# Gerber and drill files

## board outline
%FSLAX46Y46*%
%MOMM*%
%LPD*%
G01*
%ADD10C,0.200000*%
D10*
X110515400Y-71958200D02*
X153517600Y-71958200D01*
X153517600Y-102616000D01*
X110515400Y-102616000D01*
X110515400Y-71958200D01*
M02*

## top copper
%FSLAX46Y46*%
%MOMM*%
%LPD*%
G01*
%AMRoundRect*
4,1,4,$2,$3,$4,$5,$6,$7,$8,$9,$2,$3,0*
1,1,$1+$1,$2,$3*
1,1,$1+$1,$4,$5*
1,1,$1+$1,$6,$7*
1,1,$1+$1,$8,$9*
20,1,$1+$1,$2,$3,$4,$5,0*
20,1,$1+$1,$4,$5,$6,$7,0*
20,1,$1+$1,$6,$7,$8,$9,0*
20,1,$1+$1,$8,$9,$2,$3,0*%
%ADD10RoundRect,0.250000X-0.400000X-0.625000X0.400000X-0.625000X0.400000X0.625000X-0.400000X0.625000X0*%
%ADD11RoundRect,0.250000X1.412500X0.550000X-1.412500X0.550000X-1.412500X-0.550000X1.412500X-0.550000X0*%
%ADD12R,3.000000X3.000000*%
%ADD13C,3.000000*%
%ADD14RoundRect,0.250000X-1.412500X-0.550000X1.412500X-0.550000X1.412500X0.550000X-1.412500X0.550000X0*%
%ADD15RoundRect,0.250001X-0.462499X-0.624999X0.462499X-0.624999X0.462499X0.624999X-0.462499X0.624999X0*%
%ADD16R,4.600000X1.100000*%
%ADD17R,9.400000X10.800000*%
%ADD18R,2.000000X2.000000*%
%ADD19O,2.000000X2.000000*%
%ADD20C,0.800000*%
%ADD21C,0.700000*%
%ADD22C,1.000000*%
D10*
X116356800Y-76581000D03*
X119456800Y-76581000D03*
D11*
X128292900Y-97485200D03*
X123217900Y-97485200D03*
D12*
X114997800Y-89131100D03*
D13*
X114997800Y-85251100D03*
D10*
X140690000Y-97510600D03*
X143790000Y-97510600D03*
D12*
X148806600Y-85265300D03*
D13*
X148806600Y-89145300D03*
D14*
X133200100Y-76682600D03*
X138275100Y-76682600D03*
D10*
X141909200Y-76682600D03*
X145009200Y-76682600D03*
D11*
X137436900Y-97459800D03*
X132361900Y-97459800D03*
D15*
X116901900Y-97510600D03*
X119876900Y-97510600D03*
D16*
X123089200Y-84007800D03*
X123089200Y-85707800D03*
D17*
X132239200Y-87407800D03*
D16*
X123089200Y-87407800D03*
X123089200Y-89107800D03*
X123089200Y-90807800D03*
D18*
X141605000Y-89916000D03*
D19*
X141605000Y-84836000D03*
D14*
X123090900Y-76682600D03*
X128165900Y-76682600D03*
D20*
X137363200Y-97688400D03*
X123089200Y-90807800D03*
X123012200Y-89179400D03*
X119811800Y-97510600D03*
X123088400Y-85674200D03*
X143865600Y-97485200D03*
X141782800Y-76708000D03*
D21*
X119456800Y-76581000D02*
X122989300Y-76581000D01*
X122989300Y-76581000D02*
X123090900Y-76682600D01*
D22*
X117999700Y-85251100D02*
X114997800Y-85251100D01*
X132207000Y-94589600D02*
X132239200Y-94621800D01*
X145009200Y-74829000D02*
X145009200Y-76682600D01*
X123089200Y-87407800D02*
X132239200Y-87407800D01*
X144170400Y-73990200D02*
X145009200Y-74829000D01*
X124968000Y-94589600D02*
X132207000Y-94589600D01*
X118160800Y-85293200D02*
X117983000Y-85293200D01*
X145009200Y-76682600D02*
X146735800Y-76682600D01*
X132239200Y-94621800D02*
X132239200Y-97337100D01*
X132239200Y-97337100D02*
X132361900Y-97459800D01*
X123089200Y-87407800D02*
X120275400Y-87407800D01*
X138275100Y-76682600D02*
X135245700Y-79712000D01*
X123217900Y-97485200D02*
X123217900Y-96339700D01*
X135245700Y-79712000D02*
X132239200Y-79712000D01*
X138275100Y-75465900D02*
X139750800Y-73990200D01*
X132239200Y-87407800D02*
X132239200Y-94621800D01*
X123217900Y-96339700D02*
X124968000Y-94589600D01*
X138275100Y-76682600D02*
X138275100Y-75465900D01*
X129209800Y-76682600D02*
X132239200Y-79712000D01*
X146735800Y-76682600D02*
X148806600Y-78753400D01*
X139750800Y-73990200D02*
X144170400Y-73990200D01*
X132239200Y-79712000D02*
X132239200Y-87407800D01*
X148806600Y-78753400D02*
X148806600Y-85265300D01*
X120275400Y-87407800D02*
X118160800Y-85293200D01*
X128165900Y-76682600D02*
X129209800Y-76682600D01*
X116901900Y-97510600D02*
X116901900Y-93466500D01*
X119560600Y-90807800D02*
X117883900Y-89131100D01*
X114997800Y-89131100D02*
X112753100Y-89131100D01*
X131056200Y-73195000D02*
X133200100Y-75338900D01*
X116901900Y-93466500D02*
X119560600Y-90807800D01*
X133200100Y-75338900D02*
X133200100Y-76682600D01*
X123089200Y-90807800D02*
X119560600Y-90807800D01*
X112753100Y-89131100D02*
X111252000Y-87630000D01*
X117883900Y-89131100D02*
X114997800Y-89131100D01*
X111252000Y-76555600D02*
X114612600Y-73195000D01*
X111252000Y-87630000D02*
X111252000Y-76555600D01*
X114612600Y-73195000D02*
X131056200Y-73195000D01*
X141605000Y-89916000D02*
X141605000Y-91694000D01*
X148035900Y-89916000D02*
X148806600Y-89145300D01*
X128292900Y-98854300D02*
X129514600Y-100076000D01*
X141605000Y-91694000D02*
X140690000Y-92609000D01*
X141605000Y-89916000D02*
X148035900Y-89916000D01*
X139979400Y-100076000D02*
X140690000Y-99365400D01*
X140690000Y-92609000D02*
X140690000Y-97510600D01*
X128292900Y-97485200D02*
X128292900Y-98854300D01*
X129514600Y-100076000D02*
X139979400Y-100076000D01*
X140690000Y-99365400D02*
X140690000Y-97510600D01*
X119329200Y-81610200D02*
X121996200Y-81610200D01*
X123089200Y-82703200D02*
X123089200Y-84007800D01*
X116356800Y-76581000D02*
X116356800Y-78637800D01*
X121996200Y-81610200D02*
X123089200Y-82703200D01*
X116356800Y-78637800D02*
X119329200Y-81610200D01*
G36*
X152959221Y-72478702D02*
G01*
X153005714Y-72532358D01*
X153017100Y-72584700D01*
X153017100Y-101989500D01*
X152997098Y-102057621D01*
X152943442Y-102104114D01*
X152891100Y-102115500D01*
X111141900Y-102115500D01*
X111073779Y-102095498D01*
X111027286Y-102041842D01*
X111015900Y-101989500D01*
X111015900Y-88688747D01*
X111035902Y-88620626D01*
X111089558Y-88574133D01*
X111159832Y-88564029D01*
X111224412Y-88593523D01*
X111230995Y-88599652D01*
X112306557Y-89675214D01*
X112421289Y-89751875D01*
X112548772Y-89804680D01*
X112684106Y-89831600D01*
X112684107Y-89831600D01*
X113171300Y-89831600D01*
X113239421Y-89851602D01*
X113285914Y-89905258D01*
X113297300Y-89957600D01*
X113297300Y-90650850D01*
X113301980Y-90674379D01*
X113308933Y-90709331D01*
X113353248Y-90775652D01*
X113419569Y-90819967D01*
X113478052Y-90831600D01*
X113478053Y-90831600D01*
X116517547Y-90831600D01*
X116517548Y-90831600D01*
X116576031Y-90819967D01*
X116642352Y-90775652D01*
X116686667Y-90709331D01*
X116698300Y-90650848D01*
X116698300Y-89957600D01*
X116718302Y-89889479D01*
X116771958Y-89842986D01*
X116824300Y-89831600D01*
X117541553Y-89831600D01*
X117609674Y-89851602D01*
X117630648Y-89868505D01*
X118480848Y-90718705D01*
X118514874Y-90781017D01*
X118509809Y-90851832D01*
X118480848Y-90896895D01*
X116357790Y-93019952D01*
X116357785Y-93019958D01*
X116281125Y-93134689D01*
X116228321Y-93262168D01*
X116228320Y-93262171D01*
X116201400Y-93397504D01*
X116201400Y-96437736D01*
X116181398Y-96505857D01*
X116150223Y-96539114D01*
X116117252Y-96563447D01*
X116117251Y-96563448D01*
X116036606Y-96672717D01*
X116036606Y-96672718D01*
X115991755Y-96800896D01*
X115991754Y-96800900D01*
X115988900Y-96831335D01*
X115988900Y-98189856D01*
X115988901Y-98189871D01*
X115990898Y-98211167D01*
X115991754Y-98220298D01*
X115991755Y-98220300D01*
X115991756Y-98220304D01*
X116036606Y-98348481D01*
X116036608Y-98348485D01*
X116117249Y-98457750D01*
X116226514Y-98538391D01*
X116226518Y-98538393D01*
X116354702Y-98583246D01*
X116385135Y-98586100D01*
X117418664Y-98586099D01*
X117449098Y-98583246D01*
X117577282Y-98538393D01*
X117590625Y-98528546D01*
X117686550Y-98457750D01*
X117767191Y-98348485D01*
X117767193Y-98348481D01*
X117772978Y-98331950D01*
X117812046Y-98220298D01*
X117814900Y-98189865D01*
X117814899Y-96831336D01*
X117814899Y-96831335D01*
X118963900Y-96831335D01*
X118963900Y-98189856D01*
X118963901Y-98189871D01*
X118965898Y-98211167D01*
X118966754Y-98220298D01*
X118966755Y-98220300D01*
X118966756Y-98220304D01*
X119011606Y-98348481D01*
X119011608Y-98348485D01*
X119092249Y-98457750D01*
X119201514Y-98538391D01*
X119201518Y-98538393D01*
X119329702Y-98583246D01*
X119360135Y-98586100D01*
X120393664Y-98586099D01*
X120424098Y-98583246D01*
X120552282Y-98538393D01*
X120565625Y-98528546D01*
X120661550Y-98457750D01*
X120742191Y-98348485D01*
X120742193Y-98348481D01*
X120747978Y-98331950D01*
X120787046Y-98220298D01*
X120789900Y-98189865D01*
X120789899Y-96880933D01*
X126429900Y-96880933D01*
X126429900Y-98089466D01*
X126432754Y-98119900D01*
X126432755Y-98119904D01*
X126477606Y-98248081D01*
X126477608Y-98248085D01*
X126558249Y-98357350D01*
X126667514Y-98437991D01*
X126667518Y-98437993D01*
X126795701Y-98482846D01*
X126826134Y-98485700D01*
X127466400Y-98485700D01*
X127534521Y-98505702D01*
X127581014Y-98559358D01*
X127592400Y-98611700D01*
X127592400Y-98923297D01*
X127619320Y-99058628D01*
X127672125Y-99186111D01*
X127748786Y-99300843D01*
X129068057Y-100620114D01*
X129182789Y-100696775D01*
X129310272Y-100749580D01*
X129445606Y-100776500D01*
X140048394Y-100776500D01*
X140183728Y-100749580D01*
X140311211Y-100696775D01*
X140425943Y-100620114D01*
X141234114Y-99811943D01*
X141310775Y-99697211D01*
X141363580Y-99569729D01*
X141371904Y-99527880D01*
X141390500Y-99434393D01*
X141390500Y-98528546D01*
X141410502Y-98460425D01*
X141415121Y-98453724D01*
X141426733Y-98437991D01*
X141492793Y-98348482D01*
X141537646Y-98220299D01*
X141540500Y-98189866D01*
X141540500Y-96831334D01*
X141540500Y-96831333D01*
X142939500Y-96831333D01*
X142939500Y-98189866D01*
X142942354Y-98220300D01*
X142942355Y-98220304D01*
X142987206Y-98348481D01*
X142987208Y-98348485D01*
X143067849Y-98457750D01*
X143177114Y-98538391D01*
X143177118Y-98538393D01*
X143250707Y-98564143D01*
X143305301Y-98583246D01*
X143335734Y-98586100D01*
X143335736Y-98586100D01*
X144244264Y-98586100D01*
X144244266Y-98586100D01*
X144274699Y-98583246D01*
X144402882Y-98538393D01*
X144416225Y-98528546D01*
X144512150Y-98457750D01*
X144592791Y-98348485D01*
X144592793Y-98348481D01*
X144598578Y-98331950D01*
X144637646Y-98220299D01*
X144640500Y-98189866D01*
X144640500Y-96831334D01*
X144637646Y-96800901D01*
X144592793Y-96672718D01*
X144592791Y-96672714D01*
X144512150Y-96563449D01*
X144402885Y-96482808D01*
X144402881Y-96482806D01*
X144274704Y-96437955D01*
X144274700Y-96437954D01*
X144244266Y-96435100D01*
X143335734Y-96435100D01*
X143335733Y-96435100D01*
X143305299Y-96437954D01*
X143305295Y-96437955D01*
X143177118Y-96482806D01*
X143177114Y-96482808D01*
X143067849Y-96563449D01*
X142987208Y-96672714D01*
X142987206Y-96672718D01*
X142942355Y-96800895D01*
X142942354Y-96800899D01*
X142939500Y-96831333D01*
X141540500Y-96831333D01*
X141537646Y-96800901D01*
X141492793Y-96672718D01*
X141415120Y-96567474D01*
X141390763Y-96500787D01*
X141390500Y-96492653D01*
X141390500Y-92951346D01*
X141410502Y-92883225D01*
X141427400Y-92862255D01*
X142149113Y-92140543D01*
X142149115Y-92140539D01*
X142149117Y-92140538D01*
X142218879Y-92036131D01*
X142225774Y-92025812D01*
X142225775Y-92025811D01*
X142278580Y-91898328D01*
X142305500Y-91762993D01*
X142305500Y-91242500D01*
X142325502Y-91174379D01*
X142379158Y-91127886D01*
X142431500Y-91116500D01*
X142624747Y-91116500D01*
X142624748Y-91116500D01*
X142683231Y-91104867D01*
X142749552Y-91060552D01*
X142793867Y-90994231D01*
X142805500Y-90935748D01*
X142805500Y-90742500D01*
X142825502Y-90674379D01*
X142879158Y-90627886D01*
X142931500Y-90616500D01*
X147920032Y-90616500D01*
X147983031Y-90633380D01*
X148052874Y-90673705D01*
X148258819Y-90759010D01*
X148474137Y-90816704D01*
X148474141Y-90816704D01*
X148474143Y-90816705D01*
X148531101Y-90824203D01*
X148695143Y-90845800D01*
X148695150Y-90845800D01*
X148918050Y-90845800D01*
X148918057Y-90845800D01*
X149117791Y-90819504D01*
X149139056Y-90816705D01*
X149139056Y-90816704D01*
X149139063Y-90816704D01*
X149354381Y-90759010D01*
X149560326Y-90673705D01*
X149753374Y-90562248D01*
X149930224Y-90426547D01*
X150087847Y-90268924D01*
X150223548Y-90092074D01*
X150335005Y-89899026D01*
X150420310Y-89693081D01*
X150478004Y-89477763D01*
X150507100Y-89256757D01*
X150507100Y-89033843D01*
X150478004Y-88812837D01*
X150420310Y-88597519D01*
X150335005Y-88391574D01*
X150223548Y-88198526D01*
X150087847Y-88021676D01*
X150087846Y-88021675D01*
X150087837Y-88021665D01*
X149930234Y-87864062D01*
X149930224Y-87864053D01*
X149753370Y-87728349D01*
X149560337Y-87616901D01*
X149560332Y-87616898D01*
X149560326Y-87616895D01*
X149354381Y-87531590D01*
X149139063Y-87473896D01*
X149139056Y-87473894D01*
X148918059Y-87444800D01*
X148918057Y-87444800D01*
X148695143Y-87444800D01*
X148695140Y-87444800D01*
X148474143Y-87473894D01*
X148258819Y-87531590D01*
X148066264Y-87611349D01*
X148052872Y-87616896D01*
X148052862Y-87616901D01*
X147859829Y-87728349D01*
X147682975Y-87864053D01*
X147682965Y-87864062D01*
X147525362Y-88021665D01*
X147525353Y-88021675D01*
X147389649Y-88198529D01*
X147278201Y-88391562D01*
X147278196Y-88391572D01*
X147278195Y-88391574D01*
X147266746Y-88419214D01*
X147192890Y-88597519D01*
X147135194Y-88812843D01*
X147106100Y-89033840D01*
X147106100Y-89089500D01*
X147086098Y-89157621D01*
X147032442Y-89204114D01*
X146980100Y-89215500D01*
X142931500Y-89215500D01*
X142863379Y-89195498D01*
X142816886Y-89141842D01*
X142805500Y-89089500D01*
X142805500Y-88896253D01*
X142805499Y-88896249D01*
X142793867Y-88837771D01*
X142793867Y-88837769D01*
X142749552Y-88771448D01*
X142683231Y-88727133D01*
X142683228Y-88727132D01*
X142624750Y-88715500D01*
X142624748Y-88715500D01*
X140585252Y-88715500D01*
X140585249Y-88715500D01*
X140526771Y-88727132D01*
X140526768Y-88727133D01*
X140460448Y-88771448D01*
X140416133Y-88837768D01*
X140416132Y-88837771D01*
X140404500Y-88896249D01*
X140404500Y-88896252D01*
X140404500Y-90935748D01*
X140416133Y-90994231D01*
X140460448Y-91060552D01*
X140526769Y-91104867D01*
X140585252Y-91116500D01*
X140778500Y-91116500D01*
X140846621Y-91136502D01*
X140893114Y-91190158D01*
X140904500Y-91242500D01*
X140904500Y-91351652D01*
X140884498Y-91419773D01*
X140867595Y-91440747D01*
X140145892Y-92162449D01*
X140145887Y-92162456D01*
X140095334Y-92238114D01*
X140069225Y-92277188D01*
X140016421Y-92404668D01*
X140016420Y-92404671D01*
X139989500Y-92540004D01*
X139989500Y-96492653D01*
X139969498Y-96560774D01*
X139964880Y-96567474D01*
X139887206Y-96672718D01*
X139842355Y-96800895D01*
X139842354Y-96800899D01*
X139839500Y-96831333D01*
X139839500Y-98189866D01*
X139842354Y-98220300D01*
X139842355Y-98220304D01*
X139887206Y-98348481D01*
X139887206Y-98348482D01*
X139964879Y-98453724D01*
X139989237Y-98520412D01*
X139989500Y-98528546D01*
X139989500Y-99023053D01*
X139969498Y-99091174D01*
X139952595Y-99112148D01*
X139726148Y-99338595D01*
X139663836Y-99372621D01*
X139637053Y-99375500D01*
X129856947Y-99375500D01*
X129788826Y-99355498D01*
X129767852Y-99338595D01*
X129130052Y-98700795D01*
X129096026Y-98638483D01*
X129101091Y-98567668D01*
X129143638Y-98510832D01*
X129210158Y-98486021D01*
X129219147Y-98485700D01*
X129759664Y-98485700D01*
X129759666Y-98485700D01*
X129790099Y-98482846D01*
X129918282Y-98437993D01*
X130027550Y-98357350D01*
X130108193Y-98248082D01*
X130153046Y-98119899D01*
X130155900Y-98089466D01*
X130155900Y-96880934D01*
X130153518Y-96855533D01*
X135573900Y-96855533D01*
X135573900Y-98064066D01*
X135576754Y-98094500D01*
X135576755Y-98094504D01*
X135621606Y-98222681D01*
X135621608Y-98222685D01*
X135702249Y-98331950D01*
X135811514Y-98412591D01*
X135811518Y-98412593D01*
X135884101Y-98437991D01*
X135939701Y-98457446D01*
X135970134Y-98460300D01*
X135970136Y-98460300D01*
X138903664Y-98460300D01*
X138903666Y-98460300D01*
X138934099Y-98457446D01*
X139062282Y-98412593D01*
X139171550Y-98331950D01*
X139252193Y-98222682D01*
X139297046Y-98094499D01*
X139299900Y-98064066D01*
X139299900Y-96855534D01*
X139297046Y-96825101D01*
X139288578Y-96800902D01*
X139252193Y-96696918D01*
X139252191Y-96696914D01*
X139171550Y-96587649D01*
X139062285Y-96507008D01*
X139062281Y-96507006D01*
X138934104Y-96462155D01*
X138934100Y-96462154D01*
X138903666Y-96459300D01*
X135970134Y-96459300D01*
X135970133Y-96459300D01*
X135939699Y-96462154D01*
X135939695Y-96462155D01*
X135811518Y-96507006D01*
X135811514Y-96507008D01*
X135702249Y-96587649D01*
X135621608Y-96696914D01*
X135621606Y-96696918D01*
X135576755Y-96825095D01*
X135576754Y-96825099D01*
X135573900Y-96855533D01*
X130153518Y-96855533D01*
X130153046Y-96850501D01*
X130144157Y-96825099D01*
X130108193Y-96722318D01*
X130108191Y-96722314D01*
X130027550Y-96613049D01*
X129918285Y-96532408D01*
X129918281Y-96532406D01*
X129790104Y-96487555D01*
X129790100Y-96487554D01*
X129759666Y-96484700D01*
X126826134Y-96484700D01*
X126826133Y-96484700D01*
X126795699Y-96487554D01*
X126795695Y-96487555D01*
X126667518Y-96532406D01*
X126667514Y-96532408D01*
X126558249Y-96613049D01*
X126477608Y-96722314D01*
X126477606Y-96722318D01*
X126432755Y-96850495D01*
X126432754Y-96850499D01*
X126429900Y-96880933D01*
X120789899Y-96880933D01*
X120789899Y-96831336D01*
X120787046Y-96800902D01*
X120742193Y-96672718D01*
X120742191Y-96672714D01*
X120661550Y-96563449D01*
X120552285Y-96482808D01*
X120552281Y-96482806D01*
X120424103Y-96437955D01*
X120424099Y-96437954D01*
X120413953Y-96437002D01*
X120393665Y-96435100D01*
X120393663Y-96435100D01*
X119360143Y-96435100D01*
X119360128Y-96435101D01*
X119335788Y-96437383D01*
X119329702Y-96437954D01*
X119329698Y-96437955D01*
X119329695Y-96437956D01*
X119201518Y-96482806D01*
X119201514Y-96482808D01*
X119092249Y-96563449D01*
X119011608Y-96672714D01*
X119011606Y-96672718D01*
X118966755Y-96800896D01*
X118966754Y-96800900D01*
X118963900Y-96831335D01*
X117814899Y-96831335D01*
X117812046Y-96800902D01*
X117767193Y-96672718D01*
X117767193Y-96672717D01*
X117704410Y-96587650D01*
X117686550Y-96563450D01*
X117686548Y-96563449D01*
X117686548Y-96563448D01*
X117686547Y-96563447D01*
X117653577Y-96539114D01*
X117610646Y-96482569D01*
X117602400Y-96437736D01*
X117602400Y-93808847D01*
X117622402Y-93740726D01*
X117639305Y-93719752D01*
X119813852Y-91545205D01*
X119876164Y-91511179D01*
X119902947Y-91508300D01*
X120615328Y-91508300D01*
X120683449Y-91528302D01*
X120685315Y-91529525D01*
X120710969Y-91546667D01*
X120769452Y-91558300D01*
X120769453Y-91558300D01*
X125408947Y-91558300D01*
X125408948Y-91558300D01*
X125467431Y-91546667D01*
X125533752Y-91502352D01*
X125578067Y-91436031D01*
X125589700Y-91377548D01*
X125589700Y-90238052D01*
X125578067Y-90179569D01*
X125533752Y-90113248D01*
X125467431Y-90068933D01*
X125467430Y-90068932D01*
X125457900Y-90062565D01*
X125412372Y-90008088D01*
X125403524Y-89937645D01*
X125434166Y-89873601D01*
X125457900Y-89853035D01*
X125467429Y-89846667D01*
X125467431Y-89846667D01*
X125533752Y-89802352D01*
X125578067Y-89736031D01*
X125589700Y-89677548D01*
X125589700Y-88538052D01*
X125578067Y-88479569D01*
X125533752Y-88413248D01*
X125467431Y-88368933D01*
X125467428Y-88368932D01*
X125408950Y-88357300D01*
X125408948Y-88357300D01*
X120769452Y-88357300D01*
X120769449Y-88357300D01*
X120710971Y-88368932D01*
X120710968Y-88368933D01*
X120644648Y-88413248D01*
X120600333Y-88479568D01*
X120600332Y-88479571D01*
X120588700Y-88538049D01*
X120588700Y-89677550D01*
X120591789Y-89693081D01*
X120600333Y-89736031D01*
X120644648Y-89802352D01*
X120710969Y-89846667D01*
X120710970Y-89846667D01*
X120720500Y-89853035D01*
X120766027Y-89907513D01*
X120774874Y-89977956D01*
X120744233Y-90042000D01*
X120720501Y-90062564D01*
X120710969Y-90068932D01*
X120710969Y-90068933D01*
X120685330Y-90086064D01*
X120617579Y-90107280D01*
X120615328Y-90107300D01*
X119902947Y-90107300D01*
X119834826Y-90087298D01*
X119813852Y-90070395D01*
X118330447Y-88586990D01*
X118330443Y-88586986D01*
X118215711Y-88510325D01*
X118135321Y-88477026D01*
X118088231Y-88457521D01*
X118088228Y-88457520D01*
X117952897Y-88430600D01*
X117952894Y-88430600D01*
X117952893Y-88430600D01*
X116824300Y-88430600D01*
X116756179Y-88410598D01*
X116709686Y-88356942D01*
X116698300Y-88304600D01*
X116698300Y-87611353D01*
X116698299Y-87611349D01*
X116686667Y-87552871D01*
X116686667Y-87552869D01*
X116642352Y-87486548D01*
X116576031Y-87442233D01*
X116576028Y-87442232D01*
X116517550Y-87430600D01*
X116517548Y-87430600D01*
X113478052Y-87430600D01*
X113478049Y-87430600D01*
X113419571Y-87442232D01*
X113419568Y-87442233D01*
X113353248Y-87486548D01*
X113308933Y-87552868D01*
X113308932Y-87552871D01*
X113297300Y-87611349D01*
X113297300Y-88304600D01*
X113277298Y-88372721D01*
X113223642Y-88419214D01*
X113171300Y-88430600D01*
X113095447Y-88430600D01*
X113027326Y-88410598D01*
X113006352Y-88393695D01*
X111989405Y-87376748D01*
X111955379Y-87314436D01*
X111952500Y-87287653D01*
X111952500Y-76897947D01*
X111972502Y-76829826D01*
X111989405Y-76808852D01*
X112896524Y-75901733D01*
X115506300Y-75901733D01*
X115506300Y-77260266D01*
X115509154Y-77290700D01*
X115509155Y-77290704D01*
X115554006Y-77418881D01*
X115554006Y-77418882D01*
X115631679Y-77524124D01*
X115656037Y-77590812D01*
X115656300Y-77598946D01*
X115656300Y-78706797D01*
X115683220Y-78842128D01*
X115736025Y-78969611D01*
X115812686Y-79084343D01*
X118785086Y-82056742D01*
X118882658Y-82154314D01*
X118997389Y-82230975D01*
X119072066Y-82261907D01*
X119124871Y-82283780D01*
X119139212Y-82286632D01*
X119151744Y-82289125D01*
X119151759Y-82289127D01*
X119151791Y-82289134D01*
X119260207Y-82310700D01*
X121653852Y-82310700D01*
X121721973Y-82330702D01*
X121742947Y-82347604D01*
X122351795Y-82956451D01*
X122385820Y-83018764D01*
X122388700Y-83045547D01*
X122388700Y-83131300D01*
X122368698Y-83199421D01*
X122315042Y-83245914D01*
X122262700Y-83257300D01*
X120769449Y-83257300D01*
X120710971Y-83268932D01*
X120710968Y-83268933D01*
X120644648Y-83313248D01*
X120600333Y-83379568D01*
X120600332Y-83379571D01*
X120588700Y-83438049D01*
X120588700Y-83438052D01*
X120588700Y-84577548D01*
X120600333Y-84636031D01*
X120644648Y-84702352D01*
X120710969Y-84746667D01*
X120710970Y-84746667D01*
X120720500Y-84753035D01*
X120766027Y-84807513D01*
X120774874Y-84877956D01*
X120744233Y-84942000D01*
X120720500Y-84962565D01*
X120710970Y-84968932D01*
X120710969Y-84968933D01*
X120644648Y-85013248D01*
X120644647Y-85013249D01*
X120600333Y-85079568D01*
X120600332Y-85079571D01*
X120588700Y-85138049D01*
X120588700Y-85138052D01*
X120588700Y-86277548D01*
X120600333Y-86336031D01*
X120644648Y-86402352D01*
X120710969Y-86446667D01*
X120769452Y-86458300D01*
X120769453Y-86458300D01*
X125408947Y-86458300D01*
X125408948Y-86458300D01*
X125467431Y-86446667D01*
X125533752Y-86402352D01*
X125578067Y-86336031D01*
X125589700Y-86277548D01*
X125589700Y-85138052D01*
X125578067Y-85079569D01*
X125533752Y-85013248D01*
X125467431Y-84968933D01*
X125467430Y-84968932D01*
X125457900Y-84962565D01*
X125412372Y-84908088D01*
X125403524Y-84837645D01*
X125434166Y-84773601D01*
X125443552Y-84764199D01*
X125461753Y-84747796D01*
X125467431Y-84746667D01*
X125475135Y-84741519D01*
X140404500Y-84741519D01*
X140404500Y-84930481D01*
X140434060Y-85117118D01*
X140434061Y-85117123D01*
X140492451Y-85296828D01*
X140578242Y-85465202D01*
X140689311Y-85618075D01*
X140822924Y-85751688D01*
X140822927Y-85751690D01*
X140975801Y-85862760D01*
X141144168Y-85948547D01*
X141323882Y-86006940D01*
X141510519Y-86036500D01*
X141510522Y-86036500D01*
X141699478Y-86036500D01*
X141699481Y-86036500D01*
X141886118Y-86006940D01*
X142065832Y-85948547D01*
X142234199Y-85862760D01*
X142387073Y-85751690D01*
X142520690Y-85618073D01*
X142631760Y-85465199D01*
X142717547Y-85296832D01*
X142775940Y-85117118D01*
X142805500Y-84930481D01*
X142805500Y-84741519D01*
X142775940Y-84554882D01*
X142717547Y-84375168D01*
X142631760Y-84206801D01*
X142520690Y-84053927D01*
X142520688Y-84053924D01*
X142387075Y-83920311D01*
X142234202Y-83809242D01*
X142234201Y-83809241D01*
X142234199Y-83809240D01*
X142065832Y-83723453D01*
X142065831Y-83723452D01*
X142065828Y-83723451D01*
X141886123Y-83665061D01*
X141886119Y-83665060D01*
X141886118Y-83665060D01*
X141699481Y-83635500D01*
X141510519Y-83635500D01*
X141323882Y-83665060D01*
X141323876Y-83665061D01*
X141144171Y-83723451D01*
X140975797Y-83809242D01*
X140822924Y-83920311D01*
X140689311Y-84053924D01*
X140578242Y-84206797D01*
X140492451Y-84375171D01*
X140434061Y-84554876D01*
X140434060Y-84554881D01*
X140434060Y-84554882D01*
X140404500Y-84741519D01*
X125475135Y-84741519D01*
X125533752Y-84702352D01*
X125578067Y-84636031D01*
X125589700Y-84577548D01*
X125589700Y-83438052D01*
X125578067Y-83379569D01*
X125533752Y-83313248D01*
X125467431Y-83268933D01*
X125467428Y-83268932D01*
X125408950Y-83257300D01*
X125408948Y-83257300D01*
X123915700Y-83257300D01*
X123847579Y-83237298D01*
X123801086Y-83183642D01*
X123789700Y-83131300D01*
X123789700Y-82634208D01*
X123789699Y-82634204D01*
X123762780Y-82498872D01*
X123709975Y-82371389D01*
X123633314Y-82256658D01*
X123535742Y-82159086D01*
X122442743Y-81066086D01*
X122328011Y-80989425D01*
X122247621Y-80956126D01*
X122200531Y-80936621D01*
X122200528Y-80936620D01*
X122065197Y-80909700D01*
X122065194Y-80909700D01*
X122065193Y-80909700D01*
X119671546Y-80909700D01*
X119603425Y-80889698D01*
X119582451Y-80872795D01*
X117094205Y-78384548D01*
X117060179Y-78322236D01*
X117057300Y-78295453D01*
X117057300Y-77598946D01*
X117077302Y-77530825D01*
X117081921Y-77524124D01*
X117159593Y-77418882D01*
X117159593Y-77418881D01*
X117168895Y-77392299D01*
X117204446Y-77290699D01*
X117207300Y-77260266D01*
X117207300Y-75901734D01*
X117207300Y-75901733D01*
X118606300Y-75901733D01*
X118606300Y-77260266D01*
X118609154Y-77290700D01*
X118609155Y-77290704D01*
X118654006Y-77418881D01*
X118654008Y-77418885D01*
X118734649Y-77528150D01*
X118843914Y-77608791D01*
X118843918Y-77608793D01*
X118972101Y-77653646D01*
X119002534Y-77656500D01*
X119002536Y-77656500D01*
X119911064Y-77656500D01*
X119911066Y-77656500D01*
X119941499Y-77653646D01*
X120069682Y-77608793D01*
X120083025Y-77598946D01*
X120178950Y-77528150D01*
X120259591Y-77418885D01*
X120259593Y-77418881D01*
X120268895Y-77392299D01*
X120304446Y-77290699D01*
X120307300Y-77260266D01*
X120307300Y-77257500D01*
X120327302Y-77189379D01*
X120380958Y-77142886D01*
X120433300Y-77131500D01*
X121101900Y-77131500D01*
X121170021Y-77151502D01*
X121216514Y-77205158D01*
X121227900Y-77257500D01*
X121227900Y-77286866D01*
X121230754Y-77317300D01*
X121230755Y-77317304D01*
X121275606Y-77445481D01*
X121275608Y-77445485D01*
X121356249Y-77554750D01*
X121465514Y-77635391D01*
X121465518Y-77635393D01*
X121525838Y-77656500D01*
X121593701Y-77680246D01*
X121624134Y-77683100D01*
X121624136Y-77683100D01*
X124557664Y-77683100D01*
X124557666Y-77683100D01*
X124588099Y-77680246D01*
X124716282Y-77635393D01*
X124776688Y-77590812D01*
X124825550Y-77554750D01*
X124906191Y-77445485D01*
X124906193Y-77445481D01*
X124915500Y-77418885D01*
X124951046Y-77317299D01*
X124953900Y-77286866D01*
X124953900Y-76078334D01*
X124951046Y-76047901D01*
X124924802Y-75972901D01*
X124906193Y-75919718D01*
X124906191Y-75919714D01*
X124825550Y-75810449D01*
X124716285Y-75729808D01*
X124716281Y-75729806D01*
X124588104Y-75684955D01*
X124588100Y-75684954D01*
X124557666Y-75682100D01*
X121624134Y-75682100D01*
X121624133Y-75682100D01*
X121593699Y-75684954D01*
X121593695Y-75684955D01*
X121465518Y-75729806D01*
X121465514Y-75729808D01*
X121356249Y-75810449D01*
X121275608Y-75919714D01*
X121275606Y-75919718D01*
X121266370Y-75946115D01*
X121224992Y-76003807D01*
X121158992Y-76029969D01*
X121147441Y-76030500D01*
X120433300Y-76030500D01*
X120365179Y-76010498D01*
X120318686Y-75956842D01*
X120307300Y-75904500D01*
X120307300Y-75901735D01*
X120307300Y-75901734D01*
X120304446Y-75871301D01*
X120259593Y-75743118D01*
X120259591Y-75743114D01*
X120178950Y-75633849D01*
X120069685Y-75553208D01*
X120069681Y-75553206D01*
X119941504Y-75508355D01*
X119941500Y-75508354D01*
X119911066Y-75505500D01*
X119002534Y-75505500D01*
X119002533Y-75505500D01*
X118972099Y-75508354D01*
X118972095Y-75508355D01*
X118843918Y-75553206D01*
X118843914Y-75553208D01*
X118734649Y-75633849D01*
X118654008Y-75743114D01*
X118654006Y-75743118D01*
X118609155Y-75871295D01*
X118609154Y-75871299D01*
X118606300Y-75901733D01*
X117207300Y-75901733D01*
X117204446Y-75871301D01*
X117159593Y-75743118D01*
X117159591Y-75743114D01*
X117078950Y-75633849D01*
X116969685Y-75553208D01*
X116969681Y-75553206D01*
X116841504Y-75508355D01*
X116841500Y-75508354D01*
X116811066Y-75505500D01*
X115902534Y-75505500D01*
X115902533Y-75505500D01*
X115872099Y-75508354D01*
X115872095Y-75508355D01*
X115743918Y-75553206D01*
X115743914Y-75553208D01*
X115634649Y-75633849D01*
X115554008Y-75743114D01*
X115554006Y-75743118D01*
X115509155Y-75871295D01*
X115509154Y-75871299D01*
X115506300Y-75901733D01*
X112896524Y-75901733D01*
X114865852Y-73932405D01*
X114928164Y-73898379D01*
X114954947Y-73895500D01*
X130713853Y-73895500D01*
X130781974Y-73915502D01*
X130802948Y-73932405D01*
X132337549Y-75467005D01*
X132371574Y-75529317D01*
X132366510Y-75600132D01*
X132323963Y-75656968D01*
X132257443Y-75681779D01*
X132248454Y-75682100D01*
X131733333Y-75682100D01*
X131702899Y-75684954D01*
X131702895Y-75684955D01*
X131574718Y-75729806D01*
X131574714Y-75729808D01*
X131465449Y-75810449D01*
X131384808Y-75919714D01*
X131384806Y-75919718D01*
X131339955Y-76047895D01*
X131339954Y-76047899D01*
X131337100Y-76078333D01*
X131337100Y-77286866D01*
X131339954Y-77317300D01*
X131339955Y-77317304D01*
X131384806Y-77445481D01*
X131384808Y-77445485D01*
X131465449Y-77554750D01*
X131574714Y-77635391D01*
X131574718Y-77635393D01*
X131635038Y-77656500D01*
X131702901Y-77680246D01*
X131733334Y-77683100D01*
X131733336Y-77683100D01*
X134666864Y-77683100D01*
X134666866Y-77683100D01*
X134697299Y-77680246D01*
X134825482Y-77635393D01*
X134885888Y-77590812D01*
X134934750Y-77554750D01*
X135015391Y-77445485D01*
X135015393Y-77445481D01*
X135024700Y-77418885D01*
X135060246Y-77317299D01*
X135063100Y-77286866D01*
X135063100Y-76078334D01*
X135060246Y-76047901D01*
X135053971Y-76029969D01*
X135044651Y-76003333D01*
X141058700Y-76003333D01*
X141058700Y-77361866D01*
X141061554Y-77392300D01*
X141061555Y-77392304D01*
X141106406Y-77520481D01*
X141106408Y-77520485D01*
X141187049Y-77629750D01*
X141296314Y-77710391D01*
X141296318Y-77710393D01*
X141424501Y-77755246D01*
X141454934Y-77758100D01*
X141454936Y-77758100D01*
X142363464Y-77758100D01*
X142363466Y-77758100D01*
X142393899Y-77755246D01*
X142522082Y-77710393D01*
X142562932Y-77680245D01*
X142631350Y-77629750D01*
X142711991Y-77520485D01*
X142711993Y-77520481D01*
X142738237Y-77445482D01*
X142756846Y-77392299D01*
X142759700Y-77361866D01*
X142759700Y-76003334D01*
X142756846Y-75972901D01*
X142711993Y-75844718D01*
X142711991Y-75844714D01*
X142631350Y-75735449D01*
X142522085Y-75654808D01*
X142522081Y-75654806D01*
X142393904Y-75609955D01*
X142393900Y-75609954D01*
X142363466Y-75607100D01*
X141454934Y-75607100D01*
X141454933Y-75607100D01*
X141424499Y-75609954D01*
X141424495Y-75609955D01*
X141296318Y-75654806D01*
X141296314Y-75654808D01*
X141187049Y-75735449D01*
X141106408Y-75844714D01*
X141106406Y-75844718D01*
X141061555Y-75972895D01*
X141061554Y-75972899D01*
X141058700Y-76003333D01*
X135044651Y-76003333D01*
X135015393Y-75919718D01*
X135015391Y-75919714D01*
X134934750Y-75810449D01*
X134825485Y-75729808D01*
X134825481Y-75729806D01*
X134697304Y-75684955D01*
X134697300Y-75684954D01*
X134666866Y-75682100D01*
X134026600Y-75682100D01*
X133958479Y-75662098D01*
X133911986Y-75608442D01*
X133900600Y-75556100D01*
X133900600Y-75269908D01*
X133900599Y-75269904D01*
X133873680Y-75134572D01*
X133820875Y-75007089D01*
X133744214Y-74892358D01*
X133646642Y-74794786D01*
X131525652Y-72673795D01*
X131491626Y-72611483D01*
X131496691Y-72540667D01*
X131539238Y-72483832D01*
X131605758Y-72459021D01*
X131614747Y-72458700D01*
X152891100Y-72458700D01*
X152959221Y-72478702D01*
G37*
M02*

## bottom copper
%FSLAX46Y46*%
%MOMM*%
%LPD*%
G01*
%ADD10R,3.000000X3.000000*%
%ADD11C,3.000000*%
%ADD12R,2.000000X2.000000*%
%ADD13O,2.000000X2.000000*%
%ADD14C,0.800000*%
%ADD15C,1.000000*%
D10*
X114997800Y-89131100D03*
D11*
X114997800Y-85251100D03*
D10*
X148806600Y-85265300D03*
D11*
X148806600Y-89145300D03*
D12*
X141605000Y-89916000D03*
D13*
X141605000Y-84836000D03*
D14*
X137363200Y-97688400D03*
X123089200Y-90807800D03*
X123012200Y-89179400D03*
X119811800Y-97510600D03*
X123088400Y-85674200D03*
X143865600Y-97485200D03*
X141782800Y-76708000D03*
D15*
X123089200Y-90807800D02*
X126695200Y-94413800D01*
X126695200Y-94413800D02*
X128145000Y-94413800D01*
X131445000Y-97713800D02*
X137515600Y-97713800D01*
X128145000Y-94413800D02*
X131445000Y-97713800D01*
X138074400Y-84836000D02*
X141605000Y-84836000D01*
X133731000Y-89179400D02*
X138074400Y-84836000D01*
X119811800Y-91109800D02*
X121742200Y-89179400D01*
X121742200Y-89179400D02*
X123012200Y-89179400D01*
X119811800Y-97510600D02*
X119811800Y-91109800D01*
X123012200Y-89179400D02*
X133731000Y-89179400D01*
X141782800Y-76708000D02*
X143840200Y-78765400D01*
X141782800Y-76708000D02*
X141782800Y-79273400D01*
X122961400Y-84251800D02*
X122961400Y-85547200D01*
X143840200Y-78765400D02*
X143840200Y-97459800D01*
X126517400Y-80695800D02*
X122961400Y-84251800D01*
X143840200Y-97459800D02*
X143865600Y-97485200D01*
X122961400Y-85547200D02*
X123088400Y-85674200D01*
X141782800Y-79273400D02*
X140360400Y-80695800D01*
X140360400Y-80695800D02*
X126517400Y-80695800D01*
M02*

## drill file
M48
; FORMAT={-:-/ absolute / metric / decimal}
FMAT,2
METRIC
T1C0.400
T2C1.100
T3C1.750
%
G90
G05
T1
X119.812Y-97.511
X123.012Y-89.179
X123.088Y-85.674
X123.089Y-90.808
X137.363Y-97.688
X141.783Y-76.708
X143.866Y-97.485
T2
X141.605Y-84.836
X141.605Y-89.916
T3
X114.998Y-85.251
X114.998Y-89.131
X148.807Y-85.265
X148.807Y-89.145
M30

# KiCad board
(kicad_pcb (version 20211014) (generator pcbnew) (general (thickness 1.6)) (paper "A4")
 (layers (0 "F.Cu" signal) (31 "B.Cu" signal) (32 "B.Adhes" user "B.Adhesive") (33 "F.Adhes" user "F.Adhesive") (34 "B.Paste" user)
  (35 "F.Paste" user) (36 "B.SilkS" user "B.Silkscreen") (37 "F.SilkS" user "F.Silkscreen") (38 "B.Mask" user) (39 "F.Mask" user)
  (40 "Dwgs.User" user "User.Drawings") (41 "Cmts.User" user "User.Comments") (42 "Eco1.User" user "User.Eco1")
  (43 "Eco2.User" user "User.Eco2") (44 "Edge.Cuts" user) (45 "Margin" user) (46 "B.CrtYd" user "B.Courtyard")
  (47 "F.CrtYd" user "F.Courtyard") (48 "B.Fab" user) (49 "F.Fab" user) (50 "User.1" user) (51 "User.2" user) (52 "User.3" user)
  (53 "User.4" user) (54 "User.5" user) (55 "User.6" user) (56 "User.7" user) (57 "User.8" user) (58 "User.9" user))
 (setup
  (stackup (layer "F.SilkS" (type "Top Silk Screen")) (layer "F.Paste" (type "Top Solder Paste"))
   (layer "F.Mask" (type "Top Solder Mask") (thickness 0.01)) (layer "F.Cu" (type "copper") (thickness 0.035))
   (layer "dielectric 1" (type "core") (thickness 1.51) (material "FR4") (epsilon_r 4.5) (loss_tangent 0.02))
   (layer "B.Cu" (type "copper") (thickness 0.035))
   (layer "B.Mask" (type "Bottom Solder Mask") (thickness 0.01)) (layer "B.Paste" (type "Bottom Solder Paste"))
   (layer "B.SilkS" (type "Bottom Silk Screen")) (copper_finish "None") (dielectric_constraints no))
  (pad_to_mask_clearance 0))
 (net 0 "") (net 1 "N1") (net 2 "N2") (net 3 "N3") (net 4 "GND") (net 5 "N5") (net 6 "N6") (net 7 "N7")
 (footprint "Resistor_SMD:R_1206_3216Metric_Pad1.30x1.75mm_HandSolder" (layer "F.Cu") (at 117.9068 76.581)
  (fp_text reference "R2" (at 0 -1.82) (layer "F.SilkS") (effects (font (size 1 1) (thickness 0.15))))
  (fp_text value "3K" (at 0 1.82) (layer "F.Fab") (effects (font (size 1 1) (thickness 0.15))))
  (pad "1" smd roundrect (at -1.55 0) (size 1.3 1.75) (layers "F.Cu" "F.Paste" "F.Mask") (roundrect_rratio 0.1923076923) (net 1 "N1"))
  (pad "2" smd roundrect (at 1.55 0) (size 1.3 1.75) (layers "F.Cu" "F.Paste" "F.Mask") (roundrect_rratio 0.1923076923) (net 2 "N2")))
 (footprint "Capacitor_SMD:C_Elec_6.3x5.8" (layer "F.Cu") (at 125.7554 97.4852 180)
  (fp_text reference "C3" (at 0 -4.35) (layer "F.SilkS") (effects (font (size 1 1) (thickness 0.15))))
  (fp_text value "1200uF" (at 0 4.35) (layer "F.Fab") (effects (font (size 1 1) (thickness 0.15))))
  (pad "1" smd roundrect (at -2.5375 0 180) (size 3.325 1.6) (layers "F.Cu" "F.Paste" "F.Mask") (roundrect_rratio 0.15625) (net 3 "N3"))
  (pad "2" smd roundrect (at 2.5375 0 180) (size 3.325 1.6) (layers "F.Cu" "F.Paste" "F.Mask") (roundrect_rratio 0.15625) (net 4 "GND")))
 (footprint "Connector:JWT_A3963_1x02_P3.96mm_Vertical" (layer "F.Cu") (at 114.9978 89.1311 90)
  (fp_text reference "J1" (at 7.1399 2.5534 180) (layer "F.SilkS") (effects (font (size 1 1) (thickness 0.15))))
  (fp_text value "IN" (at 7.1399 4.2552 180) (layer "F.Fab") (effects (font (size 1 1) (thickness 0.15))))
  (pad "1" thru_hole rect (at 0 0 90) (size 3 3) (drill 1.75) (layers *.Cu *.Mask) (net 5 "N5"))
  (pad "2" thru_hole circle (at 3.88 0 90) (size 3 3) (drill 1.75) (layers *.Cu *.Mask) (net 4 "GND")))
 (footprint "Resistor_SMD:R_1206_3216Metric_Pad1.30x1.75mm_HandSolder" (layer "F.Cu") (at 142.24 97.5106)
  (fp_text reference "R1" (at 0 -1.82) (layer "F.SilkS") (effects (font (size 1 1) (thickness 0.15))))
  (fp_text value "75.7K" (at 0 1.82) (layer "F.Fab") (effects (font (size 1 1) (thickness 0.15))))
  (pad "1" smd roundrect (at -1.55 0) (size 1.3 1.75) (layers "F.Cu" "F.Paste" "F.Mask") (roundrect_rratio 0.1923076923) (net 3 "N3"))
  (pad "2" smd roundrect (at 1.55 0) (size 1.3 1.75) (layers "F.Cu" "F.Paste" "F.Mask") (roundrect_rratio 0.1923076923) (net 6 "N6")))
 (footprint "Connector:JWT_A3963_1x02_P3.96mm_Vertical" (layer "F.Cu") (at 148.8066 85.2653 -90)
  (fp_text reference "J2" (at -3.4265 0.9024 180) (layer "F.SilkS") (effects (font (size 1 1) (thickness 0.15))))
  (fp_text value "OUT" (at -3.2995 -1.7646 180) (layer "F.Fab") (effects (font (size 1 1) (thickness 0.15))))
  (pad "1" thru_hole rect (at 0 0 270) (size 3 3) (drill 1.75) (layers *.Cu *.Mask) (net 4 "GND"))
  (pad "2" thru_hole circle (at 3.88 0 270) (size 3 3) (drill 1.75) (layers *.Cu *.Mask) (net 3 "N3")))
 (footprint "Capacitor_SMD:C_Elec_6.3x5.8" (layer "F.Cu") (at 135.7376 76.6826)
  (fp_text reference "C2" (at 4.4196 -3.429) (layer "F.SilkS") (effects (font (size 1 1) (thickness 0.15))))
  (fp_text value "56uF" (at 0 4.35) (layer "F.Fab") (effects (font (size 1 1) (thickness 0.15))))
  (pad "1" smd roundrect (at -2.5375 0) (size 3.325 1.6) (layers "F.Cu" "F.Paste" "F.Mask") (roundrect_rratio 0.15625) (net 5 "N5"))
  (pad "2" smd roundrect (at 2.5375 0) (size 3.325 1.6) (layers "F.Cu" "F.Paste" "F.Mask") (roundrect_rratio 0.15625) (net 4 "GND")))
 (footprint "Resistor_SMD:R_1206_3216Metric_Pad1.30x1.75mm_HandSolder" (layer "F.Cu") (at 143.4592 76.6826)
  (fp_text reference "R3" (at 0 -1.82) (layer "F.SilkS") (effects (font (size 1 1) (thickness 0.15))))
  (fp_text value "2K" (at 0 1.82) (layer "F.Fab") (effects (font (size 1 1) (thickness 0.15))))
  (pad "1" smd roundrect (at -1.55 0) (size 1.3 1.75) (layers "F.Cu" "F.Paste" "F.Mask") (roundrect_rratio 0.1923076923) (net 6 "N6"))
  (pad "2" smd roundrect (at 1.55 0) (size 1.3 1.75) (layers "F.Cu" "F.Paste" "F.Mask") (roundrect_rratio 0.1923076923) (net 4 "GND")))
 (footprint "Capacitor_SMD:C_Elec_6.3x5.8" (layer "F.Cu") (at 134.8994 97.4598 180)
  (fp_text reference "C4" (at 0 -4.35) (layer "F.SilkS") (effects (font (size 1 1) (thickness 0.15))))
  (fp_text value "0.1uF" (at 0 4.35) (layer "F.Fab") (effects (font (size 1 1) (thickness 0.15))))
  (pad "1" smd roundrect (at -2.5375 0 180) (size 3.325 1.6) (layers "F.Cu" "F.Paste" "F.Mask") (roundrect_rratio 0.15625) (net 5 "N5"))
  (pad "2" smd roundrect (at 2.5375 0 180) (size 3.325 1.6) (layers "F.Cu" "F.Paste" "F.Mask") (roundrect_rratio 0.15625) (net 4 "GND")))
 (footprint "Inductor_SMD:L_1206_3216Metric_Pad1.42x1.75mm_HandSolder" (layer "F.Cu") (at 118.3894 97.5106)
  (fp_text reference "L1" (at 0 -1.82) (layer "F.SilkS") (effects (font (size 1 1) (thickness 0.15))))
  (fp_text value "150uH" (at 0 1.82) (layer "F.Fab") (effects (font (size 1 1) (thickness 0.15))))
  (pad "1" smd roundrect (at -1.4875 0) (size 1.425 1.75) (layers "F.Cu" "F.Paste" "F.Mask") (roundrect_rratio 0.1754392982) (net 5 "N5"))
  (pad "2" smd roundrect (at 1.4875 0) (size 1.425 1.75) (layers "F.Cu" "F.Paste" "F.Mask") (roundrect_rratio 0.1754392982) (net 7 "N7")))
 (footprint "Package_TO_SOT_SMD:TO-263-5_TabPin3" (layer "F.Cu") (at 128.8642 87.4078)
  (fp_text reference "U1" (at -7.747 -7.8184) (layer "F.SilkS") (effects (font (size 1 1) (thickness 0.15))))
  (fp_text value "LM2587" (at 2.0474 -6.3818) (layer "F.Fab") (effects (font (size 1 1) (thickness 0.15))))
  (pad "" smd rect (at 5.8 -2.775) (size 4.55 5.25) (layers "F.Paste"))
  (pad "" smd rect (at 0.95 2.775) (size 4.55 5.25) (layers "F.Paste"))
  (pad "" smd rect (at 5.8 2.775) (size 4.55 5.25) (layers "F.Paste"))
  (pad "" smd rect (at 0.95 -2.775) (size 4.55 5.25) (layers "F.Paste"))
  (pad "1" smd rect (at -5.775 -3.4) (size 4.6 1.1) (layers "F.Cu" "F.Paste" "F.Mask") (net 1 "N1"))
  (pad "2" smd rect (at -5.775 -1.7) (size 4.6 1.1) (layers "F.Cu" "F.Paste" "F.Mask") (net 6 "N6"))
  (pad "3" smd rect (at 3.375 0) (size 9.4 10.8) (layers "F.Cu" "F.Mask") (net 4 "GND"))
  (pad "3" smd rect (at -5.775 0) (size 4.6 1.1) (layers "F.Cu" "F.Paste" "F.Mask") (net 4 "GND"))
  (pad "4" smd rect (at -5.775 1.7) (size 4.6 1.1) (layers "F.Cu" "F.Paste" "F.Mask") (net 7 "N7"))
  (pad "5" smd rect (at -5.775 3.4) (size 4.6 1.1) (layers "F.Cu" "F.Paste" "F.Mask") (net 5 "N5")))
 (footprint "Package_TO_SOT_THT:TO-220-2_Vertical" (layer "F.Cu") (at 141.605 89.916 90)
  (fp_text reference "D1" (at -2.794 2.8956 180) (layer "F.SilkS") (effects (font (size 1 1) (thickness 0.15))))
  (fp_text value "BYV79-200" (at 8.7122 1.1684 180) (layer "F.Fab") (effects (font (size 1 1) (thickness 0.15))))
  (pad "1" thru_hole rect (at 0 0 90) (size 2 2) (drill 1.1) (layers *.Cu *.Mask) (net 3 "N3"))
  (pad "2" thru_hole oval (at 5.08 0 90) (size 2 2) (drill 1.1) (layers *.Cu *.Mask) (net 7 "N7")))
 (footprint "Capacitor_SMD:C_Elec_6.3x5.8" (layer "F.Cu") (at 125.6284 76.6826)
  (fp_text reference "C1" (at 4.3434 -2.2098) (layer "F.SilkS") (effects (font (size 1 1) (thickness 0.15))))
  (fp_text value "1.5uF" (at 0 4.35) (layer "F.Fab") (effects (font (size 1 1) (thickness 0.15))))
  (pad "1" smd roundrect (at -2.5375 0) (size 3.325 1.6) (layers "F.Cu" "F.Paste" "F.Mask") (roundrect_rratio 0.15625) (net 2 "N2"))
  (pad "2" smd roundrect (at 2.5375 0) (size 3.325 1.6) (layers "F.Cu" "F.Paste" "F.Mask") (roundrect_rratio 0.15625) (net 4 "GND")))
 (gr_rect (start 110.5154 71.9582) (end 153.5176 102.616) (layer "Edge.Cuts") (width 0.2) (fill none))
 (segment (start 119.4568 76.581) (end 122.9893 76.581) (width 0.7) (layer "F.Cu") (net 2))
 (segment (start 122.9893 76.581) (end 123.0909 76.6826) (width 0.7) (layer "F.Cu") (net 2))
 (segment (start 117.9997 85.2511) (end 114.9978 85.2511) (width 1) (layer "F.Cu") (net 4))
 (segment (start 132.207 94.5896) (end 132.2392 94.6218) (width 1) (layer "F.Cu") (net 4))
 (segment (start 145.0092 74.829) (end 145.0092 76.6826) (width 1) (layer "F.Cu") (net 4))
 (segment (start 123.0892 87.4078) (end 132.2392 87.4078) (width 1) (layer "F.Cu") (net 4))
 (segment (start 144.1704 73.9902) (end 145.0092 74.829) (width 1) (layer "F.Cu") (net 4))
 (segment (start 124.968 94.5896) (end 132.207 94.5896) (width 1) (layer "F.Cu") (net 4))
 (segment (start 118.1608 85.2932) (end 117.983 85.2932) (width 1) (layer "F.Cu") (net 4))
 (segment (start 145.0092 76.6826) (end 146.7358 76.6826) (width 1) (layer "F.Cu") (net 4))
 (segment (start 132.2392 94.6218) (end 132.2392 97.3371) (width 1) (layer "F.Cu") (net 4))
 (segment (start 132.2392 97.3371) (end 132.3619 97.4598) (width 1) (layer "F.Cu") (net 4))
 (segment (start 123.0892 87.4078) (end 120.2754 87.4078) (width 1) (layer "F.Cu") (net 4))
 (segment (start 138.2751 76.6826) (end 135.2457 79.712) (width 1) (layer "F.Cu") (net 4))
 (segment (start 123.2179 97.4852) (end 123.2179 96.3397) (width 1) (layer "F.Cu") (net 4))
 (segment (start 135.2457 79.712) (end 132.2392 79.712) (width 1) (layer "F.Cu") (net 4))
 (segment (start 138.2751 75.4659) (end 139.7508 73.9902) (width 1) (layer "F.Cu") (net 4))
 (segment (start 132.2392 87.4078) (end 132.2392 94.6218) (width 1) (layer "F.Cu") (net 4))
 (segment (start 123.2179 96.3397) (end 124.968 94.5896) (width 1) (layer "F.Cu") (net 4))
 (segment (start 138.2751 76.6826) (end 138.2751 75.4659) (width 1) (layer "F.Cu") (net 4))
 (segment (start 129.2098 76.6826) (end 132.2392 79.712) (width 1) (layer "F.Cu") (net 4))
 (segment (start 146.7358 76.6826) (end 148.8066 78.7534) (width 1) (layer "F.Cu") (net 4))
 (segment (start 139.7508 73.9902) (end 144.1704 73.9902) (width 1) (layer "F.Cu") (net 4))
 (segment (start 132.2392 79.712) (end 132.2392 87.4078) (width 1) (layer "F.Cu") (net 4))
 (segment (start 148.8066 78.7534) (end 148.8066 85.2653) (width 1) (layer "F.Cu") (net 4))
 (segment (start 120.2754 87.4078) (end 118.1608 85.2932) (width 1) (layer "F.Cu") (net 4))
 (segment (start 128.1659 76.6826) (end 129.2098 76.6826) (width 1) (layer "F.Cu") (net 4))
 (segment (start 116.9019 97.5106) (end 116.9019 93.4665) (width 1) (layer "F.Cu") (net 5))
 (segment (start 119.5606 90.8078) (end 117.8839 89.1311) (width 1) (layer "F.Cu") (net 5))
 (segment (start 114.9978 89.1311) (end 112.7531 89.1311) (width 1) (layer "F.Cu") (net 5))
 (segment (start 131.0562 73.195) (end 133.2001 75.3389) (width 1) (layer "F.Cu") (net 5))
 (segment (start 116.9019 93.4665) (end 119.5606 90.8078) (width 1) (layer "F.Cu") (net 5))
 (segment (start 133.2001 75.3389) (end 133.2001 76.6826) (width 1) (layer "F.Cu") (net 5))
 (segment (start 123.0892 90.8078) (end 119.5606 90.8078) (width 1) (layer "F.Cu") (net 5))
 (segment (start 112.7531 89.1311) (end 111.252 87.63) (width 1) (layer "F.Cu") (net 5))
 (segment (start 117.8839 89.1311) (end 114.9978 89.1311) (width 1) (layer "F.Cu") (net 5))
 (segment (start 111.252 76.5556) (end 114.6126 73.195) (width 1) (layer "F.Cu") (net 5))
 (segment (start 111.252 87.63) (end 111.252 76.5556) (width 1) (layer "F.Cu") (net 5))
 (segment (start 114.6126 73.195) (end 131.0562 73.195) (width 1) (layer "F.Cu") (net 5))
 (via (at 137.3632 97.6884) (size 0.8) (drill 0.4) (layers "F.Cu" "B.Cu") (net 5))
 (via (at 123.0892 90.8078) (size 0.8) (drill 0.4) (layers "F.Cu" "B.Cu") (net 5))
 (segment (start 123.0892 90.8078) (end 126.6952 94.4138) (width 1) (layer "B.Cu") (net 5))
 (segment (start 126.6952 94.4138) (end 128.145 94.4138) (width 1) (layer "B.Cu") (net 5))
 (segment (start 131.445 97.7138) (end 137.5156 97.7138) (width 1) (layer "B.Cu") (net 5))
 (segment (start 128.145 94.4138) (end 131.445 97.7138) (width 1) (layer "B.Cu") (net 5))
 (segment (start 141.605 89.916) (end 141.605 91.694) (width 1) (layer "F.Cu") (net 3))
 (segment (start 148.0359 89.916) (end 148.8066 89.1453) (width 1) (layer "F.Cu") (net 3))
 (segment (start 128.2929 98.8543) (end 129.5146 100.076) (width 1) (layer "F.Cu") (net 3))
 (segment (start 141.605 91.694) (end 140.69 92.609) (width 1) (layer "F.Cu") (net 3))
 (segment (start 141.605 89.916) (end 148.0359 89.916) (width 1) (layer "F.Cu") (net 3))
 (segment (start 139.9794 100.076) (end 140.69 99.3654) (width 1) (layer "F.Cu") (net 3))
 (segment (start 140.69 92.609) (end 140.69 97.5106) (width 1) (layer "F.Cu") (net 3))
 (segment (start 128.2929 97.4852) (end 128.2929 98.8543) (width 1) (layer "F.Cu") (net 3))
 (segment (start 129.5146 100.076) (end 139.9794 100.076) (width 1) (layer "F.Cu") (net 3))
 (segment (start 140.69 99.3654) (end 140.69 97.5106) (width 1) (layer "F.Cu") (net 3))
 (via (at 123.0122 89.1794) (size 0.8) (drill 0.4) (layers "F.Cu" "B.Cu") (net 7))
 (via (at 119.8118 97.5106) (size 0.8) (drill 0.4) (layers "F.Cu" "B.Cu") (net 7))
 (segment (start 138.0744 84.836) (end 141.605 84.836) (width 1) (layer "B.Cu") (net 7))
 (segment (start 133.731 89.1794) (end 138.0744 84.836) (width 1) (layer "B.Cu") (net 7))
 (segment (start 119.8118 91.1098) (end 121.7422 89.1794) (width 1) (layer "B.Cu") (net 7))
 (segment (start 121.7422 89.1794) (end 123.0122 89.1794) (width 1) (layer "B.Cu") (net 7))
 (segment (start 119.8118 97.5106) (end 119.8118 91.1098) (width 1) (layer "B.Cu") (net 7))
 (segment (start 123.0122 89.1794) (end 133.731 89.1794) (width 1) (layer "B.Cu") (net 7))
 (via (at 123.0884 85.6742) (size 0.8) (drill 0.4) (layers "F.Cu" "B.Cu") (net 6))
 (via (at 143.8656 97.4852) (size 0.8) (drill 0.4) (layers "F.Cu" "B.Cu") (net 6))
 (via (at 141.7828 76.708) (size 0.8) (drill 0.4) (layers "F.Cu" "B.Cu") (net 6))
 (segment (start 141.7828 76.708) (end 143.8402 78.7654) (width 1) (layer "B.Cu") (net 6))
 (segment (start 141.7828 76.708) (end 141.7828 79.2734) (width 1) (layer "B.Cu") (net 6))
 (segment (start 122.9614 84.2518) (end 122.9614 85.5472) (width 1) (layer "B.Cu") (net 6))
 (segment (start 143.8402 78.7654) (end 143.8402 97.4598) (width 1) (layer "B.Cu") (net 6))
 (segment (start 126.5174 80.6958) (end 122.9614 84.2518) (width 1) (layer "B.Cu") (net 6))
 (segment (start 143.8402 97.4598) (end 143.8656 97.4852) (width 1) (layer "B.Cu") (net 6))
 (segment (start 122.9614 85.5472) (end 123.0884 85.6742) (width 1) (layer "B.Cu") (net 6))
 (segment (start 141.7828 79.2734) (end 140.3604 80.6958) (width 1) (layer "B.Cu") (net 6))
 (segment (start 140.3604 80.6958) (end 126.5174 80.6958) (width 1) (layer "B.Cu") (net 6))
 (segment (start 119.3292 81.6102) (end 121.9962 81.6102) (width 1) (layer "F.Cu") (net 1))
 (segment (start 123.0892 82.7032) (end 123.0892 84.0078) (width 1) (layer "F.Cu") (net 1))
 (segment (start 116.3568 76.581) (end 116.3568 78.6378) (width 1) (layer "F.Cu") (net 1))
 (segment (start 121.9962 81.6102) (end 123.0892 82.7032) (width 1) (layer "F.Cu") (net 1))
 (segment (start 116.3568 78.6378) (end 119.3292 81.6102) (width 1) (layer "F.Cu") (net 1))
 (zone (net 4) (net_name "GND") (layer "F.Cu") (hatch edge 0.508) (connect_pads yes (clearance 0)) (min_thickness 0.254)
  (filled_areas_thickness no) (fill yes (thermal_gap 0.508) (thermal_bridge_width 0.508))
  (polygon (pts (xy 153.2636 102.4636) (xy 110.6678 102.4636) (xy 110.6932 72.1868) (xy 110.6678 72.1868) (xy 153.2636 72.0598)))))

